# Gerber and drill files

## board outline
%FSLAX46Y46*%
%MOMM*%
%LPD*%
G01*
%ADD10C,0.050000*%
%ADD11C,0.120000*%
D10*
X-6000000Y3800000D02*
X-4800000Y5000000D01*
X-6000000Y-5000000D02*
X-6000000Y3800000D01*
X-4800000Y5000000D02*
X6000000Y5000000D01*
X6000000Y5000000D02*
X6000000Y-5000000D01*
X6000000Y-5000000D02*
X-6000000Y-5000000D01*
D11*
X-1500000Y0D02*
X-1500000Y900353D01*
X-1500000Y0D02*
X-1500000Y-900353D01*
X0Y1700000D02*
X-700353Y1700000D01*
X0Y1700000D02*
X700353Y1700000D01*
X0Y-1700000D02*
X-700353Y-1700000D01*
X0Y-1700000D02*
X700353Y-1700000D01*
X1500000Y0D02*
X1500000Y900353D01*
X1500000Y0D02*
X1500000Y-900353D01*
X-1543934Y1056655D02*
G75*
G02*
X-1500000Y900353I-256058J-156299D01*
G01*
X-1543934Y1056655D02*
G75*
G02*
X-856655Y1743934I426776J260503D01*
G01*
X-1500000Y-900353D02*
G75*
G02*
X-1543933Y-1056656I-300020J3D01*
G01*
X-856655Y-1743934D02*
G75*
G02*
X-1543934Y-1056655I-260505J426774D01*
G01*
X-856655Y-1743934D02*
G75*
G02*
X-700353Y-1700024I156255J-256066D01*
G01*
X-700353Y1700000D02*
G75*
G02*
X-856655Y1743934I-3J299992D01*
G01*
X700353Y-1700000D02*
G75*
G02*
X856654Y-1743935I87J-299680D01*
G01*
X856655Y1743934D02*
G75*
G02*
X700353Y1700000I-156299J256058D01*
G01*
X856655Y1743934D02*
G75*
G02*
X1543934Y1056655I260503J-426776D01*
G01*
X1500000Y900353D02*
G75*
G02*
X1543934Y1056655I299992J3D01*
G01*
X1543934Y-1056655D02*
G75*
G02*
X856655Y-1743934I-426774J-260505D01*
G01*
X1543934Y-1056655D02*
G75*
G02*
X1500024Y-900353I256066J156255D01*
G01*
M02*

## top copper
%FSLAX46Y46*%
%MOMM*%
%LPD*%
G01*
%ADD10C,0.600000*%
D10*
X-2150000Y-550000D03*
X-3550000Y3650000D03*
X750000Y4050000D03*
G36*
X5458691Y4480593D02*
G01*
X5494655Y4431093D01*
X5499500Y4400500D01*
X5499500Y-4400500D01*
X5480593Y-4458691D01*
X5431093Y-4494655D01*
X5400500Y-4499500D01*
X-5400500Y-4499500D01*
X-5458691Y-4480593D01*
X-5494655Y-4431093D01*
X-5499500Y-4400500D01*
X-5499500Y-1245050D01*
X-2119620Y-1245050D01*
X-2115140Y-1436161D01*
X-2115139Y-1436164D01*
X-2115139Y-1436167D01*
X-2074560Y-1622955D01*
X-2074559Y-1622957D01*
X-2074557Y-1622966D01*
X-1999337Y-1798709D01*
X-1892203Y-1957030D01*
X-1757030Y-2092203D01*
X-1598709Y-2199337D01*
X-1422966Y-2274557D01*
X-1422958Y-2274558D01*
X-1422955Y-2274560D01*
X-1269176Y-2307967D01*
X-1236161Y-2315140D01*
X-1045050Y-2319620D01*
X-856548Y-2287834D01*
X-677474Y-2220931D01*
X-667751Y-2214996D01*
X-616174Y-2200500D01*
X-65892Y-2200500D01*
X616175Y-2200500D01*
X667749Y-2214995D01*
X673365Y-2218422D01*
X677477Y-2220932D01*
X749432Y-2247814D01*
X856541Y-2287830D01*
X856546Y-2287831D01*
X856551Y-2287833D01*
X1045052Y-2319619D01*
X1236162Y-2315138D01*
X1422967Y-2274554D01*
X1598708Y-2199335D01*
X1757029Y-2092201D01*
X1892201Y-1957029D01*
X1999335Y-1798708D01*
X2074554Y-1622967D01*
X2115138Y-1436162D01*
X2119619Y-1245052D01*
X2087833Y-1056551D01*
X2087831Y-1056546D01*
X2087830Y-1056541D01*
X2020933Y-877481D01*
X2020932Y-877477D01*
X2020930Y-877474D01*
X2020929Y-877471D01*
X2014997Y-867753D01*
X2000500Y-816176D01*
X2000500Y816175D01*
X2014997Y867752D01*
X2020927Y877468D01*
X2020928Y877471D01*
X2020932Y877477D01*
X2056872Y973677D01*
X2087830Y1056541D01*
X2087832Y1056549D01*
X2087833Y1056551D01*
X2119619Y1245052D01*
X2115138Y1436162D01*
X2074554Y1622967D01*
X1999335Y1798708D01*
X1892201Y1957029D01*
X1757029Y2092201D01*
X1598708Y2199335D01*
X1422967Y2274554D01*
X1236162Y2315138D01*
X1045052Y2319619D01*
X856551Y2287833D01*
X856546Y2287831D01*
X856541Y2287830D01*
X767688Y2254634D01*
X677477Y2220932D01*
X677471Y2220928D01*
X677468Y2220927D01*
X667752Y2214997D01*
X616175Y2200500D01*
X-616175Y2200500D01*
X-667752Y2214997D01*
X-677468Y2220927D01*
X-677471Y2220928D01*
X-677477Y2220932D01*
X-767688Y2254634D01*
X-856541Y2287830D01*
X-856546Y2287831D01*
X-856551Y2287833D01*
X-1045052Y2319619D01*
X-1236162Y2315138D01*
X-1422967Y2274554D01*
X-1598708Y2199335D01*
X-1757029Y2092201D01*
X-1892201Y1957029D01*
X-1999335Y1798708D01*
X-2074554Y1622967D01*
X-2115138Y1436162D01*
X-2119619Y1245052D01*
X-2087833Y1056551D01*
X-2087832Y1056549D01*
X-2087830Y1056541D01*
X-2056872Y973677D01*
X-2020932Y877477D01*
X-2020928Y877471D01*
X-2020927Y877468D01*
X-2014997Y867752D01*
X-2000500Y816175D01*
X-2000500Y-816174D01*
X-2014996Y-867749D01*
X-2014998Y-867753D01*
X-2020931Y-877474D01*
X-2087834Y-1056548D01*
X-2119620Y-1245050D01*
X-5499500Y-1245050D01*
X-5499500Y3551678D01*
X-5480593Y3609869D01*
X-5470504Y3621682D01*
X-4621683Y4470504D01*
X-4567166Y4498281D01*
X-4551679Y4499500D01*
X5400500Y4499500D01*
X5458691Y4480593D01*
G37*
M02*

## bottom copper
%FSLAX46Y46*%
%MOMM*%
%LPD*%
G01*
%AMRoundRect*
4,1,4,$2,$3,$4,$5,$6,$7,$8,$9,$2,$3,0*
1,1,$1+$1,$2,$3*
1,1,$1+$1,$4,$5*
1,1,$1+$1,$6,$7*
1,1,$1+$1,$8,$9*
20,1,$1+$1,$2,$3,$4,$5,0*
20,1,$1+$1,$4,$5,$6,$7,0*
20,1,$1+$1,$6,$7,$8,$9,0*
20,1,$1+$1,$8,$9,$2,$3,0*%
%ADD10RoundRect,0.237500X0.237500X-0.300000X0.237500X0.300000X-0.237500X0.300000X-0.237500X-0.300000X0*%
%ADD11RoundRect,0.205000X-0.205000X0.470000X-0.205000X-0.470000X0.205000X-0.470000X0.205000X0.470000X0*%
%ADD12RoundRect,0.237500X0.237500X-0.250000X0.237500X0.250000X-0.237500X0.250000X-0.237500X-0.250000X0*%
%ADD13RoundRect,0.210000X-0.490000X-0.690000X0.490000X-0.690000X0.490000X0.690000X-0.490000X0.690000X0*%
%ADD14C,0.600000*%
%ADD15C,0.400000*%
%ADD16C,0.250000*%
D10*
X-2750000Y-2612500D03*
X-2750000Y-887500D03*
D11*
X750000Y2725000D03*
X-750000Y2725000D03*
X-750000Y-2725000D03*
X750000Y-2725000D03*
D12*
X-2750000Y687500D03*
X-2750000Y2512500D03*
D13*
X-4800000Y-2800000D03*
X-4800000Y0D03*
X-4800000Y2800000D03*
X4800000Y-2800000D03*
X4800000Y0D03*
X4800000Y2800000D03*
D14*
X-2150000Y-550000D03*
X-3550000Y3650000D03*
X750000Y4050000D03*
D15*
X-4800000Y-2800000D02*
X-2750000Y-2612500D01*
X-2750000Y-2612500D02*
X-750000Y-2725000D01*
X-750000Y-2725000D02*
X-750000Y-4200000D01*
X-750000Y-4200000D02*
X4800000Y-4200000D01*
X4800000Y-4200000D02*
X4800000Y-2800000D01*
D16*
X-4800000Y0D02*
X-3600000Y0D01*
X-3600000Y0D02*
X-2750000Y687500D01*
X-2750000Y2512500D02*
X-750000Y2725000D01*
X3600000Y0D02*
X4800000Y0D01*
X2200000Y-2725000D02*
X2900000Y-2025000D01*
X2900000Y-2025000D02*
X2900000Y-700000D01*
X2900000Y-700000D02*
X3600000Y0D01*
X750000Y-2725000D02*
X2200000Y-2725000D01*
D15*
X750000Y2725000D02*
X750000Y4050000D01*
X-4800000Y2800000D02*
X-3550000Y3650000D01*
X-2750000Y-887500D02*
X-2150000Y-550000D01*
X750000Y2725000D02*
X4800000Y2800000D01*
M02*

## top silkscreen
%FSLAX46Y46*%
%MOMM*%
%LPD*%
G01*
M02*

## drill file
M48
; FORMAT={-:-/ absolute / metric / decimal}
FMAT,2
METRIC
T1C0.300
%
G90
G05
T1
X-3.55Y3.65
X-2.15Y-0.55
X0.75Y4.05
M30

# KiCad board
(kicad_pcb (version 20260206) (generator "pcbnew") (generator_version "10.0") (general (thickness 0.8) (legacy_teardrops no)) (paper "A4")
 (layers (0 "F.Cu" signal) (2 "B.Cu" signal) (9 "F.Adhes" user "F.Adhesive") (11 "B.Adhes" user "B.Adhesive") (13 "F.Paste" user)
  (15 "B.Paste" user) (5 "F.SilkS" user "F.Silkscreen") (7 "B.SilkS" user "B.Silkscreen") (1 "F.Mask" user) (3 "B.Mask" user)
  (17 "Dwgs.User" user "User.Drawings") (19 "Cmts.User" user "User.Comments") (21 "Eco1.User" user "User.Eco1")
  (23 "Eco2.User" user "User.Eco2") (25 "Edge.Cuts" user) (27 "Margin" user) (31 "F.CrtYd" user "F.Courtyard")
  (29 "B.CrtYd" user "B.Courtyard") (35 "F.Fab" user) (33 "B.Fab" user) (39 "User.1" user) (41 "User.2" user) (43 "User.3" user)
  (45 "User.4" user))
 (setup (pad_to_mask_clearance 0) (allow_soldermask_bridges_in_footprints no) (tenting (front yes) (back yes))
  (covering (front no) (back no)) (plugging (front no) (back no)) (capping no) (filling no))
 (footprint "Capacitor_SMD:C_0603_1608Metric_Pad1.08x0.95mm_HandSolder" (layer "B.Cu") (at -2.75 1.75 90)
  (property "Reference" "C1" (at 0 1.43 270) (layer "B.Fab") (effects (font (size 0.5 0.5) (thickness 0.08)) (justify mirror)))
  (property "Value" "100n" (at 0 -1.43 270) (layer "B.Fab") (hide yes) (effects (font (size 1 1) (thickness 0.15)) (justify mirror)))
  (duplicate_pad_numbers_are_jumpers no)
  (pad "1" smd roundrect (at -0.8625 0 90) (size 1.075 0.95) (layers "B.Cu" "B.Mask" "B.Paste") (roundrect_rratio 0.25) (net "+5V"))
  (pad "2" smd roundrect (at 0.8625 0 90) (size 1.075 0.95) (layers "B.Cu" "B.Mask" "B.Paste") (roundrect_rratio 0.25) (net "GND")))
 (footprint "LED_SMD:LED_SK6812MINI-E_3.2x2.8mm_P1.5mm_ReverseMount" (layer "B.Cu") (at 0 0 -90)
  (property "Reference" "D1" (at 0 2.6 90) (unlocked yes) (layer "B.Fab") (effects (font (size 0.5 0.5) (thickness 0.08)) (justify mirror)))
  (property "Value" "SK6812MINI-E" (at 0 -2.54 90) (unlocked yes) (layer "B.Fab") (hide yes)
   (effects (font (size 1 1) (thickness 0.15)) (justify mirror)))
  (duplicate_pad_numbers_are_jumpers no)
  (fp_line (start 0 1.5) (end -0.900353 1.5) (stroke (width 0.12) (type solid)) (layer "Edge.Cuts"))
  (fp_line (start 0 1.5) (end 0.900353 1.5) (stroke (width 0.12) (type solid)) (layer "Edge.Cuts"))
  (fp_line (start -1.7 0) (end -1.7 0.700353) (stroke (width 0.12) (type solid)) (layer "Edge.Cuts"))
  (fp_line (start -1.7 0) (end -1.7 -0.700353) (stroke (width 0.12) (type solid)) (layer "Edge.Cuts"))
  (fp_line (start 1.7 0) (end 1.7 0.700353) (stroke (width 0.12) (type solid)) (layer "Edge.Cuts"))
  (fp_line (start 1.7 0) (end 1.7 -0.700353) (stroke (width 0.12) (type solid)) (layer "Edge.Cuts"))
  (fp_line (start 0 -1.5) (end -0.900353 -1.5) (stroke (width 0.12) (type solid)) (layer "Edge.Cuts"))
  (fp_line (start 0 -1.5) (end 0.900353 -1.5) (stroke (width 0.12) (type solid)) (layer "Edge.Cuts"))
  (fp_arc (start -1.056655 1.543934) (mid -0.981533 1.511192) (end -0.900353 1.5) (stroke (width 0.12) (type solid)) (layer "Edge.Cuts"))
  (fp_arc (start -1.056655 1.543934) (mid -1.670711 1.470711) (end -1.743934 0.856655) (stroke (width 0.12) (type solid))
   (layer "Edge.Cuts"))
  (fp_arc (start 0.900353 1.5) (mid 0.981532 1.511193) (end 1.056655 1.543934) (stroke (width 0.12) (type solid)) (layer "Edge.Cuts"))
  (fp_arc (start 1.743934 0.856655) (mid 1.670713 1.470713) (end 1.056655 1.543934) (stroke (width 0.12) (type solid)) (layer "Edge.Cuts"))
  (fp_arc (start 1.743934 0.856655) (mid 1.711191 0.781533) (end 1.7 0.700353) (stroke (width 0.12) (type solid)) (layer "Edge.Cuts"))
  (fp_arc (start -1.7 0.700353) (mid -1.711192 0.781533) (end -1.743934 0.856655) (stroke (width 0.12) (type solid)) (layer "Edge.Cuts"))
  (fp_arc (start 1.7 -0.700353) (mid 1.711181 -0.781538) (end 1.743934 -0.856655) (stroke (width 0.12) (type solid)) (layer "Edge.Cuts"))
  (fp_arc (start -1.743934 -0.856655) (mid -1.711192 -0.781533) (end -1.7 -0.700353) (stroke (width 0.12) (type solid)) (layer "Edge.Cuts"))
  (fp_arc (start -1.743934 -0.856655) (mid -1.670711 -1.470711) (end -1.056655 -1.543934) (stroke (width 0.12) (type solid))
   (layer "Edge.Cuts"))
  (fp_arc (start -0.900353 -1.5) (mid -0.981533 -1.511192) (end -1.056655 -1.543934) (stroke (width 0.12) (type solid)) (layer "Edge.Cuts"))
  (fp_arc (start 1.056655 -1.543934) (mid 1.670711 -1.470711) (end 1.743934 -0.856655) (stroke (width 0.12) (type solid))
   (layer "Edge.Cuts"))
  (fp_arc (start 1.056655 -1.543934) (mid 0.981533 -1.511191) (end 0.900353 -1.5) (stroke (width 0.12) (type solid)) (layer "Edge.Cuts"))
  (pad "1" smd roundrect (at -2.725 -0.75 270) (size 1.35 0.82) (layers "B.Cu" "B.Mask" "B.Paste") (roundrect_rratio 0.25) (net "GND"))
  (pad "2" smd roundrect (at -2.725 0.75 270) (size 1.35 0.82) (layers "B.Cu" "B.Mask" "B.Paste") (roundrect_rratio 0.25) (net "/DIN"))
  (pad "3" smd roundrect (at 2.725 0.75 270) (size 1.35 0.82) (layers "B.Cu" "B.Mask" "B.Paste") (roundrect_rratio 0.25) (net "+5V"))
  (pad "4" smd roundrect (at 2.725 -0.75 270) (size 1.35 0.82) (layers "B.Cu" "B.Mask" "B.Paste") (roundrect_rratio 0.25) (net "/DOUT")))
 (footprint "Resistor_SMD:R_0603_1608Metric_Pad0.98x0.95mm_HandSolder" (layer "B.Cu") (at -2.75 -1.6 90)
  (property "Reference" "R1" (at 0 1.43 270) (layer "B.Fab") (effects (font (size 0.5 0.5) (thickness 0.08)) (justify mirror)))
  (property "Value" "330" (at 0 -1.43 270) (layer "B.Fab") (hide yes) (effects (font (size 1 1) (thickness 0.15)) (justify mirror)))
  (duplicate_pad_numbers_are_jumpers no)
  (pad "1" smd roundrect (at -0.9125 0 90) (size 0.975 0.95) (layers "B.Cu" "B.Mask" "B.Paste") (roundrect_rratio 0.25) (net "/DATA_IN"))
  (pad "2" smd roundrect (at 0.9125 0 90) (size 0.975 0.95) (layers "B.Cu" "B.Mask" "B.Paste") (roundrect_rratio 0.25) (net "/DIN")))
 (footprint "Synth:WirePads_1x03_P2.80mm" (layer "B.Cu") (at -4.8 0)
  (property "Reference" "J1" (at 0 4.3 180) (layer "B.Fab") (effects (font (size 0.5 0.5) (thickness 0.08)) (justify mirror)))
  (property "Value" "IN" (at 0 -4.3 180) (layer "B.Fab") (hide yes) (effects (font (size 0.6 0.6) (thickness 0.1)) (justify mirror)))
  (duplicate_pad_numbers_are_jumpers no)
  (pad "1" smd roundrect (at 0 2.8) (size 1.4 1.8) (layers "B.Cu" "B.Mask" "B.Paste") (roundrect_rratio 0.15) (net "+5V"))
  (pad "2" smd roundrect (at 0 0) (size 1.4 1.8) (layers "B.Cu" "B.Mask" "B.Paste") (roundrect_rratio 0.15) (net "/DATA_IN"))
  (pad "3" smd roundrect (at 0 -2.8) (size 1.4 1.8) (layers "B.Cu" "B.Mask" "B.Paste") (roundrect_rratio 0.15) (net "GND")))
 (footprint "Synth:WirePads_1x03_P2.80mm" (layer "B.Cu") (at 4.8 0)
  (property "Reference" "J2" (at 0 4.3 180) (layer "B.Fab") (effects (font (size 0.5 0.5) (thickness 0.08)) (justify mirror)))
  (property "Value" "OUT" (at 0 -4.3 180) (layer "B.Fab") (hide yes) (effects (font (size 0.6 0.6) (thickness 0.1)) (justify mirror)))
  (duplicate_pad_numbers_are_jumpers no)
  (pad "1" smd roundrect (at 0 2.8) (size 1.4 1.8) (layers "B.Cu" "B.Mask" "B.Paste") (roundrect_rratio 0.15) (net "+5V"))
  (pad "2" smd roundrect (at 0 0) (size 1.4 1.8) (layers "B.Cu" "B.Mask" "B.Paste") (roundrect_rratio 0.15) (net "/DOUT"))
  (pad "3" smd roundrect (at 0 -2.8) (size 1.4 1.8) (layers "B.Cu" "B.Mask" "B.Paste") (roundrect_rratio 0.15) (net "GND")))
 (gr_line (start -6 -3.8) (end -4.8 -5) (stroke (width 0.05) (type default)) (layer "Edge.Cuts"))
 (gr_line (start -6 5) (end -6 -3.8) (stroke (width 0.05) (type default)) (layer "Edge.Cuts"))
 (gr_line (start -4.8 -5) (end 6 -5) (stroke (width 0.05) (type default)) (layer "Edge.Cuts"))
 (gr_line (start 6 -5) (end 6 5) (stroke (width 0.05) (type default)) (layer "Edge.Cuts"))
 (gr_line (start 6 5) (end -6 5) (stroke (width 0.05) (type default)) (layer "Edge.Cuts"))
 (segment (start -4.8 2.8) (end -2.75 2.6125) (width 0.4) (layer "B.Cu") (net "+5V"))
 (segment (start -2.75 2.6125) (end -0.75 2.725) (width 0.4) (layer "B.Cu") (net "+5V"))
 (segment (start -0.75 2.725) (end -0.75 4.2) (width 0.4) (layer "B.Cu") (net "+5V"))
 (segment (start -0.75 4.2) (end 4.8 4.2) (width 0.4) (layer "B.Cu") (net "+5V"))
 (segment (start 4.8 4.2) (end 4.8 2.8) (width 0.4) (layer "B.Cu") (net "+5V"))
 (segment (start -4.8 0) (end -3.6 0) (width 0.25) (layer "B.Cu") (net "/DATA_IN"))
 (segment (start -3.6 0) (end -2.75 -0.6875) (width 0.25) (layer "B.Cu") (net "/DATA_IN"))
 (segment (start -2.75 -2.5125) (end -0.75 -2.725) (width 0.25) (layer "B.Cu") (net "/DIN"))
 (segment (start 3.6 0) (end 4.8 0) (width 0.25) (layer "B.Cu") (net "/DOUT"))
 (segment (start 2.2 2.725) (end 2.9 2.025) (width 0.25) (layer "B.Cu") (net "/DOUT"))
 (segment (start 2.9 2.025) (end 2.9 0.7) (width 0.25) (layer "B.Cu") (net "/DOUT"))
 (segment (start 2.9 0.7) (end 3.6 0) (width 0.25) (layer "B.Cu") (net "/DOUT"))
 (segment (start 0.75 2.725) (end 2.2 2.725) (width 0.25) (layer "B.Cu") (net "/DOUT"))
 (via (at -2.15 0.55) (size 0.6) (drill 0.3) (layers "F.Cu" "B.Cu") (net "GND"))
 (via (at -3.55 -3.65) (size 0.6) (drill 0.3) (layers "F.Cu" "B.Cu") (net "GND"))
 (via (at 0.75 -4.05) (size 0.6) (drill 0.3) (layers "F.Cu" "B.Cu") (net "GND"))
 (segment (start 0.75 -2.725) (end 0.75 -4.05) (width 0.4) (layer "B.Cu") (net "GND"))
 (segment (start -4.8 -2.8) (end -3.55 -3.65) (width 0.4) (layer "B.Cu") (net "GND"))
 (segment (start -2.75 0.8875) (end -2.15 0.55) (width 0.4) (layer "B.Cu") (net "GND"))
 (segment (start 0.75 -2.725) (end 4.8 -2.8) (width 0.4) (layer "B.Cu") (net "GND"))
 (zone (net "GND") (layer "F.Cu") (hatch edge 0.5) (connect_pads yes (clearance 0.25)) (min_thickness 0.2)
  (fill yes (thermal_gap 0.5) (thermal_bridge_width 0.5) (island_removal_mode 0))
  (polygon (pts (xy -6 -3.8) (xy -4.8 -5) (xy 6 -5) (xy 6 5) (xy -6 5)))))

